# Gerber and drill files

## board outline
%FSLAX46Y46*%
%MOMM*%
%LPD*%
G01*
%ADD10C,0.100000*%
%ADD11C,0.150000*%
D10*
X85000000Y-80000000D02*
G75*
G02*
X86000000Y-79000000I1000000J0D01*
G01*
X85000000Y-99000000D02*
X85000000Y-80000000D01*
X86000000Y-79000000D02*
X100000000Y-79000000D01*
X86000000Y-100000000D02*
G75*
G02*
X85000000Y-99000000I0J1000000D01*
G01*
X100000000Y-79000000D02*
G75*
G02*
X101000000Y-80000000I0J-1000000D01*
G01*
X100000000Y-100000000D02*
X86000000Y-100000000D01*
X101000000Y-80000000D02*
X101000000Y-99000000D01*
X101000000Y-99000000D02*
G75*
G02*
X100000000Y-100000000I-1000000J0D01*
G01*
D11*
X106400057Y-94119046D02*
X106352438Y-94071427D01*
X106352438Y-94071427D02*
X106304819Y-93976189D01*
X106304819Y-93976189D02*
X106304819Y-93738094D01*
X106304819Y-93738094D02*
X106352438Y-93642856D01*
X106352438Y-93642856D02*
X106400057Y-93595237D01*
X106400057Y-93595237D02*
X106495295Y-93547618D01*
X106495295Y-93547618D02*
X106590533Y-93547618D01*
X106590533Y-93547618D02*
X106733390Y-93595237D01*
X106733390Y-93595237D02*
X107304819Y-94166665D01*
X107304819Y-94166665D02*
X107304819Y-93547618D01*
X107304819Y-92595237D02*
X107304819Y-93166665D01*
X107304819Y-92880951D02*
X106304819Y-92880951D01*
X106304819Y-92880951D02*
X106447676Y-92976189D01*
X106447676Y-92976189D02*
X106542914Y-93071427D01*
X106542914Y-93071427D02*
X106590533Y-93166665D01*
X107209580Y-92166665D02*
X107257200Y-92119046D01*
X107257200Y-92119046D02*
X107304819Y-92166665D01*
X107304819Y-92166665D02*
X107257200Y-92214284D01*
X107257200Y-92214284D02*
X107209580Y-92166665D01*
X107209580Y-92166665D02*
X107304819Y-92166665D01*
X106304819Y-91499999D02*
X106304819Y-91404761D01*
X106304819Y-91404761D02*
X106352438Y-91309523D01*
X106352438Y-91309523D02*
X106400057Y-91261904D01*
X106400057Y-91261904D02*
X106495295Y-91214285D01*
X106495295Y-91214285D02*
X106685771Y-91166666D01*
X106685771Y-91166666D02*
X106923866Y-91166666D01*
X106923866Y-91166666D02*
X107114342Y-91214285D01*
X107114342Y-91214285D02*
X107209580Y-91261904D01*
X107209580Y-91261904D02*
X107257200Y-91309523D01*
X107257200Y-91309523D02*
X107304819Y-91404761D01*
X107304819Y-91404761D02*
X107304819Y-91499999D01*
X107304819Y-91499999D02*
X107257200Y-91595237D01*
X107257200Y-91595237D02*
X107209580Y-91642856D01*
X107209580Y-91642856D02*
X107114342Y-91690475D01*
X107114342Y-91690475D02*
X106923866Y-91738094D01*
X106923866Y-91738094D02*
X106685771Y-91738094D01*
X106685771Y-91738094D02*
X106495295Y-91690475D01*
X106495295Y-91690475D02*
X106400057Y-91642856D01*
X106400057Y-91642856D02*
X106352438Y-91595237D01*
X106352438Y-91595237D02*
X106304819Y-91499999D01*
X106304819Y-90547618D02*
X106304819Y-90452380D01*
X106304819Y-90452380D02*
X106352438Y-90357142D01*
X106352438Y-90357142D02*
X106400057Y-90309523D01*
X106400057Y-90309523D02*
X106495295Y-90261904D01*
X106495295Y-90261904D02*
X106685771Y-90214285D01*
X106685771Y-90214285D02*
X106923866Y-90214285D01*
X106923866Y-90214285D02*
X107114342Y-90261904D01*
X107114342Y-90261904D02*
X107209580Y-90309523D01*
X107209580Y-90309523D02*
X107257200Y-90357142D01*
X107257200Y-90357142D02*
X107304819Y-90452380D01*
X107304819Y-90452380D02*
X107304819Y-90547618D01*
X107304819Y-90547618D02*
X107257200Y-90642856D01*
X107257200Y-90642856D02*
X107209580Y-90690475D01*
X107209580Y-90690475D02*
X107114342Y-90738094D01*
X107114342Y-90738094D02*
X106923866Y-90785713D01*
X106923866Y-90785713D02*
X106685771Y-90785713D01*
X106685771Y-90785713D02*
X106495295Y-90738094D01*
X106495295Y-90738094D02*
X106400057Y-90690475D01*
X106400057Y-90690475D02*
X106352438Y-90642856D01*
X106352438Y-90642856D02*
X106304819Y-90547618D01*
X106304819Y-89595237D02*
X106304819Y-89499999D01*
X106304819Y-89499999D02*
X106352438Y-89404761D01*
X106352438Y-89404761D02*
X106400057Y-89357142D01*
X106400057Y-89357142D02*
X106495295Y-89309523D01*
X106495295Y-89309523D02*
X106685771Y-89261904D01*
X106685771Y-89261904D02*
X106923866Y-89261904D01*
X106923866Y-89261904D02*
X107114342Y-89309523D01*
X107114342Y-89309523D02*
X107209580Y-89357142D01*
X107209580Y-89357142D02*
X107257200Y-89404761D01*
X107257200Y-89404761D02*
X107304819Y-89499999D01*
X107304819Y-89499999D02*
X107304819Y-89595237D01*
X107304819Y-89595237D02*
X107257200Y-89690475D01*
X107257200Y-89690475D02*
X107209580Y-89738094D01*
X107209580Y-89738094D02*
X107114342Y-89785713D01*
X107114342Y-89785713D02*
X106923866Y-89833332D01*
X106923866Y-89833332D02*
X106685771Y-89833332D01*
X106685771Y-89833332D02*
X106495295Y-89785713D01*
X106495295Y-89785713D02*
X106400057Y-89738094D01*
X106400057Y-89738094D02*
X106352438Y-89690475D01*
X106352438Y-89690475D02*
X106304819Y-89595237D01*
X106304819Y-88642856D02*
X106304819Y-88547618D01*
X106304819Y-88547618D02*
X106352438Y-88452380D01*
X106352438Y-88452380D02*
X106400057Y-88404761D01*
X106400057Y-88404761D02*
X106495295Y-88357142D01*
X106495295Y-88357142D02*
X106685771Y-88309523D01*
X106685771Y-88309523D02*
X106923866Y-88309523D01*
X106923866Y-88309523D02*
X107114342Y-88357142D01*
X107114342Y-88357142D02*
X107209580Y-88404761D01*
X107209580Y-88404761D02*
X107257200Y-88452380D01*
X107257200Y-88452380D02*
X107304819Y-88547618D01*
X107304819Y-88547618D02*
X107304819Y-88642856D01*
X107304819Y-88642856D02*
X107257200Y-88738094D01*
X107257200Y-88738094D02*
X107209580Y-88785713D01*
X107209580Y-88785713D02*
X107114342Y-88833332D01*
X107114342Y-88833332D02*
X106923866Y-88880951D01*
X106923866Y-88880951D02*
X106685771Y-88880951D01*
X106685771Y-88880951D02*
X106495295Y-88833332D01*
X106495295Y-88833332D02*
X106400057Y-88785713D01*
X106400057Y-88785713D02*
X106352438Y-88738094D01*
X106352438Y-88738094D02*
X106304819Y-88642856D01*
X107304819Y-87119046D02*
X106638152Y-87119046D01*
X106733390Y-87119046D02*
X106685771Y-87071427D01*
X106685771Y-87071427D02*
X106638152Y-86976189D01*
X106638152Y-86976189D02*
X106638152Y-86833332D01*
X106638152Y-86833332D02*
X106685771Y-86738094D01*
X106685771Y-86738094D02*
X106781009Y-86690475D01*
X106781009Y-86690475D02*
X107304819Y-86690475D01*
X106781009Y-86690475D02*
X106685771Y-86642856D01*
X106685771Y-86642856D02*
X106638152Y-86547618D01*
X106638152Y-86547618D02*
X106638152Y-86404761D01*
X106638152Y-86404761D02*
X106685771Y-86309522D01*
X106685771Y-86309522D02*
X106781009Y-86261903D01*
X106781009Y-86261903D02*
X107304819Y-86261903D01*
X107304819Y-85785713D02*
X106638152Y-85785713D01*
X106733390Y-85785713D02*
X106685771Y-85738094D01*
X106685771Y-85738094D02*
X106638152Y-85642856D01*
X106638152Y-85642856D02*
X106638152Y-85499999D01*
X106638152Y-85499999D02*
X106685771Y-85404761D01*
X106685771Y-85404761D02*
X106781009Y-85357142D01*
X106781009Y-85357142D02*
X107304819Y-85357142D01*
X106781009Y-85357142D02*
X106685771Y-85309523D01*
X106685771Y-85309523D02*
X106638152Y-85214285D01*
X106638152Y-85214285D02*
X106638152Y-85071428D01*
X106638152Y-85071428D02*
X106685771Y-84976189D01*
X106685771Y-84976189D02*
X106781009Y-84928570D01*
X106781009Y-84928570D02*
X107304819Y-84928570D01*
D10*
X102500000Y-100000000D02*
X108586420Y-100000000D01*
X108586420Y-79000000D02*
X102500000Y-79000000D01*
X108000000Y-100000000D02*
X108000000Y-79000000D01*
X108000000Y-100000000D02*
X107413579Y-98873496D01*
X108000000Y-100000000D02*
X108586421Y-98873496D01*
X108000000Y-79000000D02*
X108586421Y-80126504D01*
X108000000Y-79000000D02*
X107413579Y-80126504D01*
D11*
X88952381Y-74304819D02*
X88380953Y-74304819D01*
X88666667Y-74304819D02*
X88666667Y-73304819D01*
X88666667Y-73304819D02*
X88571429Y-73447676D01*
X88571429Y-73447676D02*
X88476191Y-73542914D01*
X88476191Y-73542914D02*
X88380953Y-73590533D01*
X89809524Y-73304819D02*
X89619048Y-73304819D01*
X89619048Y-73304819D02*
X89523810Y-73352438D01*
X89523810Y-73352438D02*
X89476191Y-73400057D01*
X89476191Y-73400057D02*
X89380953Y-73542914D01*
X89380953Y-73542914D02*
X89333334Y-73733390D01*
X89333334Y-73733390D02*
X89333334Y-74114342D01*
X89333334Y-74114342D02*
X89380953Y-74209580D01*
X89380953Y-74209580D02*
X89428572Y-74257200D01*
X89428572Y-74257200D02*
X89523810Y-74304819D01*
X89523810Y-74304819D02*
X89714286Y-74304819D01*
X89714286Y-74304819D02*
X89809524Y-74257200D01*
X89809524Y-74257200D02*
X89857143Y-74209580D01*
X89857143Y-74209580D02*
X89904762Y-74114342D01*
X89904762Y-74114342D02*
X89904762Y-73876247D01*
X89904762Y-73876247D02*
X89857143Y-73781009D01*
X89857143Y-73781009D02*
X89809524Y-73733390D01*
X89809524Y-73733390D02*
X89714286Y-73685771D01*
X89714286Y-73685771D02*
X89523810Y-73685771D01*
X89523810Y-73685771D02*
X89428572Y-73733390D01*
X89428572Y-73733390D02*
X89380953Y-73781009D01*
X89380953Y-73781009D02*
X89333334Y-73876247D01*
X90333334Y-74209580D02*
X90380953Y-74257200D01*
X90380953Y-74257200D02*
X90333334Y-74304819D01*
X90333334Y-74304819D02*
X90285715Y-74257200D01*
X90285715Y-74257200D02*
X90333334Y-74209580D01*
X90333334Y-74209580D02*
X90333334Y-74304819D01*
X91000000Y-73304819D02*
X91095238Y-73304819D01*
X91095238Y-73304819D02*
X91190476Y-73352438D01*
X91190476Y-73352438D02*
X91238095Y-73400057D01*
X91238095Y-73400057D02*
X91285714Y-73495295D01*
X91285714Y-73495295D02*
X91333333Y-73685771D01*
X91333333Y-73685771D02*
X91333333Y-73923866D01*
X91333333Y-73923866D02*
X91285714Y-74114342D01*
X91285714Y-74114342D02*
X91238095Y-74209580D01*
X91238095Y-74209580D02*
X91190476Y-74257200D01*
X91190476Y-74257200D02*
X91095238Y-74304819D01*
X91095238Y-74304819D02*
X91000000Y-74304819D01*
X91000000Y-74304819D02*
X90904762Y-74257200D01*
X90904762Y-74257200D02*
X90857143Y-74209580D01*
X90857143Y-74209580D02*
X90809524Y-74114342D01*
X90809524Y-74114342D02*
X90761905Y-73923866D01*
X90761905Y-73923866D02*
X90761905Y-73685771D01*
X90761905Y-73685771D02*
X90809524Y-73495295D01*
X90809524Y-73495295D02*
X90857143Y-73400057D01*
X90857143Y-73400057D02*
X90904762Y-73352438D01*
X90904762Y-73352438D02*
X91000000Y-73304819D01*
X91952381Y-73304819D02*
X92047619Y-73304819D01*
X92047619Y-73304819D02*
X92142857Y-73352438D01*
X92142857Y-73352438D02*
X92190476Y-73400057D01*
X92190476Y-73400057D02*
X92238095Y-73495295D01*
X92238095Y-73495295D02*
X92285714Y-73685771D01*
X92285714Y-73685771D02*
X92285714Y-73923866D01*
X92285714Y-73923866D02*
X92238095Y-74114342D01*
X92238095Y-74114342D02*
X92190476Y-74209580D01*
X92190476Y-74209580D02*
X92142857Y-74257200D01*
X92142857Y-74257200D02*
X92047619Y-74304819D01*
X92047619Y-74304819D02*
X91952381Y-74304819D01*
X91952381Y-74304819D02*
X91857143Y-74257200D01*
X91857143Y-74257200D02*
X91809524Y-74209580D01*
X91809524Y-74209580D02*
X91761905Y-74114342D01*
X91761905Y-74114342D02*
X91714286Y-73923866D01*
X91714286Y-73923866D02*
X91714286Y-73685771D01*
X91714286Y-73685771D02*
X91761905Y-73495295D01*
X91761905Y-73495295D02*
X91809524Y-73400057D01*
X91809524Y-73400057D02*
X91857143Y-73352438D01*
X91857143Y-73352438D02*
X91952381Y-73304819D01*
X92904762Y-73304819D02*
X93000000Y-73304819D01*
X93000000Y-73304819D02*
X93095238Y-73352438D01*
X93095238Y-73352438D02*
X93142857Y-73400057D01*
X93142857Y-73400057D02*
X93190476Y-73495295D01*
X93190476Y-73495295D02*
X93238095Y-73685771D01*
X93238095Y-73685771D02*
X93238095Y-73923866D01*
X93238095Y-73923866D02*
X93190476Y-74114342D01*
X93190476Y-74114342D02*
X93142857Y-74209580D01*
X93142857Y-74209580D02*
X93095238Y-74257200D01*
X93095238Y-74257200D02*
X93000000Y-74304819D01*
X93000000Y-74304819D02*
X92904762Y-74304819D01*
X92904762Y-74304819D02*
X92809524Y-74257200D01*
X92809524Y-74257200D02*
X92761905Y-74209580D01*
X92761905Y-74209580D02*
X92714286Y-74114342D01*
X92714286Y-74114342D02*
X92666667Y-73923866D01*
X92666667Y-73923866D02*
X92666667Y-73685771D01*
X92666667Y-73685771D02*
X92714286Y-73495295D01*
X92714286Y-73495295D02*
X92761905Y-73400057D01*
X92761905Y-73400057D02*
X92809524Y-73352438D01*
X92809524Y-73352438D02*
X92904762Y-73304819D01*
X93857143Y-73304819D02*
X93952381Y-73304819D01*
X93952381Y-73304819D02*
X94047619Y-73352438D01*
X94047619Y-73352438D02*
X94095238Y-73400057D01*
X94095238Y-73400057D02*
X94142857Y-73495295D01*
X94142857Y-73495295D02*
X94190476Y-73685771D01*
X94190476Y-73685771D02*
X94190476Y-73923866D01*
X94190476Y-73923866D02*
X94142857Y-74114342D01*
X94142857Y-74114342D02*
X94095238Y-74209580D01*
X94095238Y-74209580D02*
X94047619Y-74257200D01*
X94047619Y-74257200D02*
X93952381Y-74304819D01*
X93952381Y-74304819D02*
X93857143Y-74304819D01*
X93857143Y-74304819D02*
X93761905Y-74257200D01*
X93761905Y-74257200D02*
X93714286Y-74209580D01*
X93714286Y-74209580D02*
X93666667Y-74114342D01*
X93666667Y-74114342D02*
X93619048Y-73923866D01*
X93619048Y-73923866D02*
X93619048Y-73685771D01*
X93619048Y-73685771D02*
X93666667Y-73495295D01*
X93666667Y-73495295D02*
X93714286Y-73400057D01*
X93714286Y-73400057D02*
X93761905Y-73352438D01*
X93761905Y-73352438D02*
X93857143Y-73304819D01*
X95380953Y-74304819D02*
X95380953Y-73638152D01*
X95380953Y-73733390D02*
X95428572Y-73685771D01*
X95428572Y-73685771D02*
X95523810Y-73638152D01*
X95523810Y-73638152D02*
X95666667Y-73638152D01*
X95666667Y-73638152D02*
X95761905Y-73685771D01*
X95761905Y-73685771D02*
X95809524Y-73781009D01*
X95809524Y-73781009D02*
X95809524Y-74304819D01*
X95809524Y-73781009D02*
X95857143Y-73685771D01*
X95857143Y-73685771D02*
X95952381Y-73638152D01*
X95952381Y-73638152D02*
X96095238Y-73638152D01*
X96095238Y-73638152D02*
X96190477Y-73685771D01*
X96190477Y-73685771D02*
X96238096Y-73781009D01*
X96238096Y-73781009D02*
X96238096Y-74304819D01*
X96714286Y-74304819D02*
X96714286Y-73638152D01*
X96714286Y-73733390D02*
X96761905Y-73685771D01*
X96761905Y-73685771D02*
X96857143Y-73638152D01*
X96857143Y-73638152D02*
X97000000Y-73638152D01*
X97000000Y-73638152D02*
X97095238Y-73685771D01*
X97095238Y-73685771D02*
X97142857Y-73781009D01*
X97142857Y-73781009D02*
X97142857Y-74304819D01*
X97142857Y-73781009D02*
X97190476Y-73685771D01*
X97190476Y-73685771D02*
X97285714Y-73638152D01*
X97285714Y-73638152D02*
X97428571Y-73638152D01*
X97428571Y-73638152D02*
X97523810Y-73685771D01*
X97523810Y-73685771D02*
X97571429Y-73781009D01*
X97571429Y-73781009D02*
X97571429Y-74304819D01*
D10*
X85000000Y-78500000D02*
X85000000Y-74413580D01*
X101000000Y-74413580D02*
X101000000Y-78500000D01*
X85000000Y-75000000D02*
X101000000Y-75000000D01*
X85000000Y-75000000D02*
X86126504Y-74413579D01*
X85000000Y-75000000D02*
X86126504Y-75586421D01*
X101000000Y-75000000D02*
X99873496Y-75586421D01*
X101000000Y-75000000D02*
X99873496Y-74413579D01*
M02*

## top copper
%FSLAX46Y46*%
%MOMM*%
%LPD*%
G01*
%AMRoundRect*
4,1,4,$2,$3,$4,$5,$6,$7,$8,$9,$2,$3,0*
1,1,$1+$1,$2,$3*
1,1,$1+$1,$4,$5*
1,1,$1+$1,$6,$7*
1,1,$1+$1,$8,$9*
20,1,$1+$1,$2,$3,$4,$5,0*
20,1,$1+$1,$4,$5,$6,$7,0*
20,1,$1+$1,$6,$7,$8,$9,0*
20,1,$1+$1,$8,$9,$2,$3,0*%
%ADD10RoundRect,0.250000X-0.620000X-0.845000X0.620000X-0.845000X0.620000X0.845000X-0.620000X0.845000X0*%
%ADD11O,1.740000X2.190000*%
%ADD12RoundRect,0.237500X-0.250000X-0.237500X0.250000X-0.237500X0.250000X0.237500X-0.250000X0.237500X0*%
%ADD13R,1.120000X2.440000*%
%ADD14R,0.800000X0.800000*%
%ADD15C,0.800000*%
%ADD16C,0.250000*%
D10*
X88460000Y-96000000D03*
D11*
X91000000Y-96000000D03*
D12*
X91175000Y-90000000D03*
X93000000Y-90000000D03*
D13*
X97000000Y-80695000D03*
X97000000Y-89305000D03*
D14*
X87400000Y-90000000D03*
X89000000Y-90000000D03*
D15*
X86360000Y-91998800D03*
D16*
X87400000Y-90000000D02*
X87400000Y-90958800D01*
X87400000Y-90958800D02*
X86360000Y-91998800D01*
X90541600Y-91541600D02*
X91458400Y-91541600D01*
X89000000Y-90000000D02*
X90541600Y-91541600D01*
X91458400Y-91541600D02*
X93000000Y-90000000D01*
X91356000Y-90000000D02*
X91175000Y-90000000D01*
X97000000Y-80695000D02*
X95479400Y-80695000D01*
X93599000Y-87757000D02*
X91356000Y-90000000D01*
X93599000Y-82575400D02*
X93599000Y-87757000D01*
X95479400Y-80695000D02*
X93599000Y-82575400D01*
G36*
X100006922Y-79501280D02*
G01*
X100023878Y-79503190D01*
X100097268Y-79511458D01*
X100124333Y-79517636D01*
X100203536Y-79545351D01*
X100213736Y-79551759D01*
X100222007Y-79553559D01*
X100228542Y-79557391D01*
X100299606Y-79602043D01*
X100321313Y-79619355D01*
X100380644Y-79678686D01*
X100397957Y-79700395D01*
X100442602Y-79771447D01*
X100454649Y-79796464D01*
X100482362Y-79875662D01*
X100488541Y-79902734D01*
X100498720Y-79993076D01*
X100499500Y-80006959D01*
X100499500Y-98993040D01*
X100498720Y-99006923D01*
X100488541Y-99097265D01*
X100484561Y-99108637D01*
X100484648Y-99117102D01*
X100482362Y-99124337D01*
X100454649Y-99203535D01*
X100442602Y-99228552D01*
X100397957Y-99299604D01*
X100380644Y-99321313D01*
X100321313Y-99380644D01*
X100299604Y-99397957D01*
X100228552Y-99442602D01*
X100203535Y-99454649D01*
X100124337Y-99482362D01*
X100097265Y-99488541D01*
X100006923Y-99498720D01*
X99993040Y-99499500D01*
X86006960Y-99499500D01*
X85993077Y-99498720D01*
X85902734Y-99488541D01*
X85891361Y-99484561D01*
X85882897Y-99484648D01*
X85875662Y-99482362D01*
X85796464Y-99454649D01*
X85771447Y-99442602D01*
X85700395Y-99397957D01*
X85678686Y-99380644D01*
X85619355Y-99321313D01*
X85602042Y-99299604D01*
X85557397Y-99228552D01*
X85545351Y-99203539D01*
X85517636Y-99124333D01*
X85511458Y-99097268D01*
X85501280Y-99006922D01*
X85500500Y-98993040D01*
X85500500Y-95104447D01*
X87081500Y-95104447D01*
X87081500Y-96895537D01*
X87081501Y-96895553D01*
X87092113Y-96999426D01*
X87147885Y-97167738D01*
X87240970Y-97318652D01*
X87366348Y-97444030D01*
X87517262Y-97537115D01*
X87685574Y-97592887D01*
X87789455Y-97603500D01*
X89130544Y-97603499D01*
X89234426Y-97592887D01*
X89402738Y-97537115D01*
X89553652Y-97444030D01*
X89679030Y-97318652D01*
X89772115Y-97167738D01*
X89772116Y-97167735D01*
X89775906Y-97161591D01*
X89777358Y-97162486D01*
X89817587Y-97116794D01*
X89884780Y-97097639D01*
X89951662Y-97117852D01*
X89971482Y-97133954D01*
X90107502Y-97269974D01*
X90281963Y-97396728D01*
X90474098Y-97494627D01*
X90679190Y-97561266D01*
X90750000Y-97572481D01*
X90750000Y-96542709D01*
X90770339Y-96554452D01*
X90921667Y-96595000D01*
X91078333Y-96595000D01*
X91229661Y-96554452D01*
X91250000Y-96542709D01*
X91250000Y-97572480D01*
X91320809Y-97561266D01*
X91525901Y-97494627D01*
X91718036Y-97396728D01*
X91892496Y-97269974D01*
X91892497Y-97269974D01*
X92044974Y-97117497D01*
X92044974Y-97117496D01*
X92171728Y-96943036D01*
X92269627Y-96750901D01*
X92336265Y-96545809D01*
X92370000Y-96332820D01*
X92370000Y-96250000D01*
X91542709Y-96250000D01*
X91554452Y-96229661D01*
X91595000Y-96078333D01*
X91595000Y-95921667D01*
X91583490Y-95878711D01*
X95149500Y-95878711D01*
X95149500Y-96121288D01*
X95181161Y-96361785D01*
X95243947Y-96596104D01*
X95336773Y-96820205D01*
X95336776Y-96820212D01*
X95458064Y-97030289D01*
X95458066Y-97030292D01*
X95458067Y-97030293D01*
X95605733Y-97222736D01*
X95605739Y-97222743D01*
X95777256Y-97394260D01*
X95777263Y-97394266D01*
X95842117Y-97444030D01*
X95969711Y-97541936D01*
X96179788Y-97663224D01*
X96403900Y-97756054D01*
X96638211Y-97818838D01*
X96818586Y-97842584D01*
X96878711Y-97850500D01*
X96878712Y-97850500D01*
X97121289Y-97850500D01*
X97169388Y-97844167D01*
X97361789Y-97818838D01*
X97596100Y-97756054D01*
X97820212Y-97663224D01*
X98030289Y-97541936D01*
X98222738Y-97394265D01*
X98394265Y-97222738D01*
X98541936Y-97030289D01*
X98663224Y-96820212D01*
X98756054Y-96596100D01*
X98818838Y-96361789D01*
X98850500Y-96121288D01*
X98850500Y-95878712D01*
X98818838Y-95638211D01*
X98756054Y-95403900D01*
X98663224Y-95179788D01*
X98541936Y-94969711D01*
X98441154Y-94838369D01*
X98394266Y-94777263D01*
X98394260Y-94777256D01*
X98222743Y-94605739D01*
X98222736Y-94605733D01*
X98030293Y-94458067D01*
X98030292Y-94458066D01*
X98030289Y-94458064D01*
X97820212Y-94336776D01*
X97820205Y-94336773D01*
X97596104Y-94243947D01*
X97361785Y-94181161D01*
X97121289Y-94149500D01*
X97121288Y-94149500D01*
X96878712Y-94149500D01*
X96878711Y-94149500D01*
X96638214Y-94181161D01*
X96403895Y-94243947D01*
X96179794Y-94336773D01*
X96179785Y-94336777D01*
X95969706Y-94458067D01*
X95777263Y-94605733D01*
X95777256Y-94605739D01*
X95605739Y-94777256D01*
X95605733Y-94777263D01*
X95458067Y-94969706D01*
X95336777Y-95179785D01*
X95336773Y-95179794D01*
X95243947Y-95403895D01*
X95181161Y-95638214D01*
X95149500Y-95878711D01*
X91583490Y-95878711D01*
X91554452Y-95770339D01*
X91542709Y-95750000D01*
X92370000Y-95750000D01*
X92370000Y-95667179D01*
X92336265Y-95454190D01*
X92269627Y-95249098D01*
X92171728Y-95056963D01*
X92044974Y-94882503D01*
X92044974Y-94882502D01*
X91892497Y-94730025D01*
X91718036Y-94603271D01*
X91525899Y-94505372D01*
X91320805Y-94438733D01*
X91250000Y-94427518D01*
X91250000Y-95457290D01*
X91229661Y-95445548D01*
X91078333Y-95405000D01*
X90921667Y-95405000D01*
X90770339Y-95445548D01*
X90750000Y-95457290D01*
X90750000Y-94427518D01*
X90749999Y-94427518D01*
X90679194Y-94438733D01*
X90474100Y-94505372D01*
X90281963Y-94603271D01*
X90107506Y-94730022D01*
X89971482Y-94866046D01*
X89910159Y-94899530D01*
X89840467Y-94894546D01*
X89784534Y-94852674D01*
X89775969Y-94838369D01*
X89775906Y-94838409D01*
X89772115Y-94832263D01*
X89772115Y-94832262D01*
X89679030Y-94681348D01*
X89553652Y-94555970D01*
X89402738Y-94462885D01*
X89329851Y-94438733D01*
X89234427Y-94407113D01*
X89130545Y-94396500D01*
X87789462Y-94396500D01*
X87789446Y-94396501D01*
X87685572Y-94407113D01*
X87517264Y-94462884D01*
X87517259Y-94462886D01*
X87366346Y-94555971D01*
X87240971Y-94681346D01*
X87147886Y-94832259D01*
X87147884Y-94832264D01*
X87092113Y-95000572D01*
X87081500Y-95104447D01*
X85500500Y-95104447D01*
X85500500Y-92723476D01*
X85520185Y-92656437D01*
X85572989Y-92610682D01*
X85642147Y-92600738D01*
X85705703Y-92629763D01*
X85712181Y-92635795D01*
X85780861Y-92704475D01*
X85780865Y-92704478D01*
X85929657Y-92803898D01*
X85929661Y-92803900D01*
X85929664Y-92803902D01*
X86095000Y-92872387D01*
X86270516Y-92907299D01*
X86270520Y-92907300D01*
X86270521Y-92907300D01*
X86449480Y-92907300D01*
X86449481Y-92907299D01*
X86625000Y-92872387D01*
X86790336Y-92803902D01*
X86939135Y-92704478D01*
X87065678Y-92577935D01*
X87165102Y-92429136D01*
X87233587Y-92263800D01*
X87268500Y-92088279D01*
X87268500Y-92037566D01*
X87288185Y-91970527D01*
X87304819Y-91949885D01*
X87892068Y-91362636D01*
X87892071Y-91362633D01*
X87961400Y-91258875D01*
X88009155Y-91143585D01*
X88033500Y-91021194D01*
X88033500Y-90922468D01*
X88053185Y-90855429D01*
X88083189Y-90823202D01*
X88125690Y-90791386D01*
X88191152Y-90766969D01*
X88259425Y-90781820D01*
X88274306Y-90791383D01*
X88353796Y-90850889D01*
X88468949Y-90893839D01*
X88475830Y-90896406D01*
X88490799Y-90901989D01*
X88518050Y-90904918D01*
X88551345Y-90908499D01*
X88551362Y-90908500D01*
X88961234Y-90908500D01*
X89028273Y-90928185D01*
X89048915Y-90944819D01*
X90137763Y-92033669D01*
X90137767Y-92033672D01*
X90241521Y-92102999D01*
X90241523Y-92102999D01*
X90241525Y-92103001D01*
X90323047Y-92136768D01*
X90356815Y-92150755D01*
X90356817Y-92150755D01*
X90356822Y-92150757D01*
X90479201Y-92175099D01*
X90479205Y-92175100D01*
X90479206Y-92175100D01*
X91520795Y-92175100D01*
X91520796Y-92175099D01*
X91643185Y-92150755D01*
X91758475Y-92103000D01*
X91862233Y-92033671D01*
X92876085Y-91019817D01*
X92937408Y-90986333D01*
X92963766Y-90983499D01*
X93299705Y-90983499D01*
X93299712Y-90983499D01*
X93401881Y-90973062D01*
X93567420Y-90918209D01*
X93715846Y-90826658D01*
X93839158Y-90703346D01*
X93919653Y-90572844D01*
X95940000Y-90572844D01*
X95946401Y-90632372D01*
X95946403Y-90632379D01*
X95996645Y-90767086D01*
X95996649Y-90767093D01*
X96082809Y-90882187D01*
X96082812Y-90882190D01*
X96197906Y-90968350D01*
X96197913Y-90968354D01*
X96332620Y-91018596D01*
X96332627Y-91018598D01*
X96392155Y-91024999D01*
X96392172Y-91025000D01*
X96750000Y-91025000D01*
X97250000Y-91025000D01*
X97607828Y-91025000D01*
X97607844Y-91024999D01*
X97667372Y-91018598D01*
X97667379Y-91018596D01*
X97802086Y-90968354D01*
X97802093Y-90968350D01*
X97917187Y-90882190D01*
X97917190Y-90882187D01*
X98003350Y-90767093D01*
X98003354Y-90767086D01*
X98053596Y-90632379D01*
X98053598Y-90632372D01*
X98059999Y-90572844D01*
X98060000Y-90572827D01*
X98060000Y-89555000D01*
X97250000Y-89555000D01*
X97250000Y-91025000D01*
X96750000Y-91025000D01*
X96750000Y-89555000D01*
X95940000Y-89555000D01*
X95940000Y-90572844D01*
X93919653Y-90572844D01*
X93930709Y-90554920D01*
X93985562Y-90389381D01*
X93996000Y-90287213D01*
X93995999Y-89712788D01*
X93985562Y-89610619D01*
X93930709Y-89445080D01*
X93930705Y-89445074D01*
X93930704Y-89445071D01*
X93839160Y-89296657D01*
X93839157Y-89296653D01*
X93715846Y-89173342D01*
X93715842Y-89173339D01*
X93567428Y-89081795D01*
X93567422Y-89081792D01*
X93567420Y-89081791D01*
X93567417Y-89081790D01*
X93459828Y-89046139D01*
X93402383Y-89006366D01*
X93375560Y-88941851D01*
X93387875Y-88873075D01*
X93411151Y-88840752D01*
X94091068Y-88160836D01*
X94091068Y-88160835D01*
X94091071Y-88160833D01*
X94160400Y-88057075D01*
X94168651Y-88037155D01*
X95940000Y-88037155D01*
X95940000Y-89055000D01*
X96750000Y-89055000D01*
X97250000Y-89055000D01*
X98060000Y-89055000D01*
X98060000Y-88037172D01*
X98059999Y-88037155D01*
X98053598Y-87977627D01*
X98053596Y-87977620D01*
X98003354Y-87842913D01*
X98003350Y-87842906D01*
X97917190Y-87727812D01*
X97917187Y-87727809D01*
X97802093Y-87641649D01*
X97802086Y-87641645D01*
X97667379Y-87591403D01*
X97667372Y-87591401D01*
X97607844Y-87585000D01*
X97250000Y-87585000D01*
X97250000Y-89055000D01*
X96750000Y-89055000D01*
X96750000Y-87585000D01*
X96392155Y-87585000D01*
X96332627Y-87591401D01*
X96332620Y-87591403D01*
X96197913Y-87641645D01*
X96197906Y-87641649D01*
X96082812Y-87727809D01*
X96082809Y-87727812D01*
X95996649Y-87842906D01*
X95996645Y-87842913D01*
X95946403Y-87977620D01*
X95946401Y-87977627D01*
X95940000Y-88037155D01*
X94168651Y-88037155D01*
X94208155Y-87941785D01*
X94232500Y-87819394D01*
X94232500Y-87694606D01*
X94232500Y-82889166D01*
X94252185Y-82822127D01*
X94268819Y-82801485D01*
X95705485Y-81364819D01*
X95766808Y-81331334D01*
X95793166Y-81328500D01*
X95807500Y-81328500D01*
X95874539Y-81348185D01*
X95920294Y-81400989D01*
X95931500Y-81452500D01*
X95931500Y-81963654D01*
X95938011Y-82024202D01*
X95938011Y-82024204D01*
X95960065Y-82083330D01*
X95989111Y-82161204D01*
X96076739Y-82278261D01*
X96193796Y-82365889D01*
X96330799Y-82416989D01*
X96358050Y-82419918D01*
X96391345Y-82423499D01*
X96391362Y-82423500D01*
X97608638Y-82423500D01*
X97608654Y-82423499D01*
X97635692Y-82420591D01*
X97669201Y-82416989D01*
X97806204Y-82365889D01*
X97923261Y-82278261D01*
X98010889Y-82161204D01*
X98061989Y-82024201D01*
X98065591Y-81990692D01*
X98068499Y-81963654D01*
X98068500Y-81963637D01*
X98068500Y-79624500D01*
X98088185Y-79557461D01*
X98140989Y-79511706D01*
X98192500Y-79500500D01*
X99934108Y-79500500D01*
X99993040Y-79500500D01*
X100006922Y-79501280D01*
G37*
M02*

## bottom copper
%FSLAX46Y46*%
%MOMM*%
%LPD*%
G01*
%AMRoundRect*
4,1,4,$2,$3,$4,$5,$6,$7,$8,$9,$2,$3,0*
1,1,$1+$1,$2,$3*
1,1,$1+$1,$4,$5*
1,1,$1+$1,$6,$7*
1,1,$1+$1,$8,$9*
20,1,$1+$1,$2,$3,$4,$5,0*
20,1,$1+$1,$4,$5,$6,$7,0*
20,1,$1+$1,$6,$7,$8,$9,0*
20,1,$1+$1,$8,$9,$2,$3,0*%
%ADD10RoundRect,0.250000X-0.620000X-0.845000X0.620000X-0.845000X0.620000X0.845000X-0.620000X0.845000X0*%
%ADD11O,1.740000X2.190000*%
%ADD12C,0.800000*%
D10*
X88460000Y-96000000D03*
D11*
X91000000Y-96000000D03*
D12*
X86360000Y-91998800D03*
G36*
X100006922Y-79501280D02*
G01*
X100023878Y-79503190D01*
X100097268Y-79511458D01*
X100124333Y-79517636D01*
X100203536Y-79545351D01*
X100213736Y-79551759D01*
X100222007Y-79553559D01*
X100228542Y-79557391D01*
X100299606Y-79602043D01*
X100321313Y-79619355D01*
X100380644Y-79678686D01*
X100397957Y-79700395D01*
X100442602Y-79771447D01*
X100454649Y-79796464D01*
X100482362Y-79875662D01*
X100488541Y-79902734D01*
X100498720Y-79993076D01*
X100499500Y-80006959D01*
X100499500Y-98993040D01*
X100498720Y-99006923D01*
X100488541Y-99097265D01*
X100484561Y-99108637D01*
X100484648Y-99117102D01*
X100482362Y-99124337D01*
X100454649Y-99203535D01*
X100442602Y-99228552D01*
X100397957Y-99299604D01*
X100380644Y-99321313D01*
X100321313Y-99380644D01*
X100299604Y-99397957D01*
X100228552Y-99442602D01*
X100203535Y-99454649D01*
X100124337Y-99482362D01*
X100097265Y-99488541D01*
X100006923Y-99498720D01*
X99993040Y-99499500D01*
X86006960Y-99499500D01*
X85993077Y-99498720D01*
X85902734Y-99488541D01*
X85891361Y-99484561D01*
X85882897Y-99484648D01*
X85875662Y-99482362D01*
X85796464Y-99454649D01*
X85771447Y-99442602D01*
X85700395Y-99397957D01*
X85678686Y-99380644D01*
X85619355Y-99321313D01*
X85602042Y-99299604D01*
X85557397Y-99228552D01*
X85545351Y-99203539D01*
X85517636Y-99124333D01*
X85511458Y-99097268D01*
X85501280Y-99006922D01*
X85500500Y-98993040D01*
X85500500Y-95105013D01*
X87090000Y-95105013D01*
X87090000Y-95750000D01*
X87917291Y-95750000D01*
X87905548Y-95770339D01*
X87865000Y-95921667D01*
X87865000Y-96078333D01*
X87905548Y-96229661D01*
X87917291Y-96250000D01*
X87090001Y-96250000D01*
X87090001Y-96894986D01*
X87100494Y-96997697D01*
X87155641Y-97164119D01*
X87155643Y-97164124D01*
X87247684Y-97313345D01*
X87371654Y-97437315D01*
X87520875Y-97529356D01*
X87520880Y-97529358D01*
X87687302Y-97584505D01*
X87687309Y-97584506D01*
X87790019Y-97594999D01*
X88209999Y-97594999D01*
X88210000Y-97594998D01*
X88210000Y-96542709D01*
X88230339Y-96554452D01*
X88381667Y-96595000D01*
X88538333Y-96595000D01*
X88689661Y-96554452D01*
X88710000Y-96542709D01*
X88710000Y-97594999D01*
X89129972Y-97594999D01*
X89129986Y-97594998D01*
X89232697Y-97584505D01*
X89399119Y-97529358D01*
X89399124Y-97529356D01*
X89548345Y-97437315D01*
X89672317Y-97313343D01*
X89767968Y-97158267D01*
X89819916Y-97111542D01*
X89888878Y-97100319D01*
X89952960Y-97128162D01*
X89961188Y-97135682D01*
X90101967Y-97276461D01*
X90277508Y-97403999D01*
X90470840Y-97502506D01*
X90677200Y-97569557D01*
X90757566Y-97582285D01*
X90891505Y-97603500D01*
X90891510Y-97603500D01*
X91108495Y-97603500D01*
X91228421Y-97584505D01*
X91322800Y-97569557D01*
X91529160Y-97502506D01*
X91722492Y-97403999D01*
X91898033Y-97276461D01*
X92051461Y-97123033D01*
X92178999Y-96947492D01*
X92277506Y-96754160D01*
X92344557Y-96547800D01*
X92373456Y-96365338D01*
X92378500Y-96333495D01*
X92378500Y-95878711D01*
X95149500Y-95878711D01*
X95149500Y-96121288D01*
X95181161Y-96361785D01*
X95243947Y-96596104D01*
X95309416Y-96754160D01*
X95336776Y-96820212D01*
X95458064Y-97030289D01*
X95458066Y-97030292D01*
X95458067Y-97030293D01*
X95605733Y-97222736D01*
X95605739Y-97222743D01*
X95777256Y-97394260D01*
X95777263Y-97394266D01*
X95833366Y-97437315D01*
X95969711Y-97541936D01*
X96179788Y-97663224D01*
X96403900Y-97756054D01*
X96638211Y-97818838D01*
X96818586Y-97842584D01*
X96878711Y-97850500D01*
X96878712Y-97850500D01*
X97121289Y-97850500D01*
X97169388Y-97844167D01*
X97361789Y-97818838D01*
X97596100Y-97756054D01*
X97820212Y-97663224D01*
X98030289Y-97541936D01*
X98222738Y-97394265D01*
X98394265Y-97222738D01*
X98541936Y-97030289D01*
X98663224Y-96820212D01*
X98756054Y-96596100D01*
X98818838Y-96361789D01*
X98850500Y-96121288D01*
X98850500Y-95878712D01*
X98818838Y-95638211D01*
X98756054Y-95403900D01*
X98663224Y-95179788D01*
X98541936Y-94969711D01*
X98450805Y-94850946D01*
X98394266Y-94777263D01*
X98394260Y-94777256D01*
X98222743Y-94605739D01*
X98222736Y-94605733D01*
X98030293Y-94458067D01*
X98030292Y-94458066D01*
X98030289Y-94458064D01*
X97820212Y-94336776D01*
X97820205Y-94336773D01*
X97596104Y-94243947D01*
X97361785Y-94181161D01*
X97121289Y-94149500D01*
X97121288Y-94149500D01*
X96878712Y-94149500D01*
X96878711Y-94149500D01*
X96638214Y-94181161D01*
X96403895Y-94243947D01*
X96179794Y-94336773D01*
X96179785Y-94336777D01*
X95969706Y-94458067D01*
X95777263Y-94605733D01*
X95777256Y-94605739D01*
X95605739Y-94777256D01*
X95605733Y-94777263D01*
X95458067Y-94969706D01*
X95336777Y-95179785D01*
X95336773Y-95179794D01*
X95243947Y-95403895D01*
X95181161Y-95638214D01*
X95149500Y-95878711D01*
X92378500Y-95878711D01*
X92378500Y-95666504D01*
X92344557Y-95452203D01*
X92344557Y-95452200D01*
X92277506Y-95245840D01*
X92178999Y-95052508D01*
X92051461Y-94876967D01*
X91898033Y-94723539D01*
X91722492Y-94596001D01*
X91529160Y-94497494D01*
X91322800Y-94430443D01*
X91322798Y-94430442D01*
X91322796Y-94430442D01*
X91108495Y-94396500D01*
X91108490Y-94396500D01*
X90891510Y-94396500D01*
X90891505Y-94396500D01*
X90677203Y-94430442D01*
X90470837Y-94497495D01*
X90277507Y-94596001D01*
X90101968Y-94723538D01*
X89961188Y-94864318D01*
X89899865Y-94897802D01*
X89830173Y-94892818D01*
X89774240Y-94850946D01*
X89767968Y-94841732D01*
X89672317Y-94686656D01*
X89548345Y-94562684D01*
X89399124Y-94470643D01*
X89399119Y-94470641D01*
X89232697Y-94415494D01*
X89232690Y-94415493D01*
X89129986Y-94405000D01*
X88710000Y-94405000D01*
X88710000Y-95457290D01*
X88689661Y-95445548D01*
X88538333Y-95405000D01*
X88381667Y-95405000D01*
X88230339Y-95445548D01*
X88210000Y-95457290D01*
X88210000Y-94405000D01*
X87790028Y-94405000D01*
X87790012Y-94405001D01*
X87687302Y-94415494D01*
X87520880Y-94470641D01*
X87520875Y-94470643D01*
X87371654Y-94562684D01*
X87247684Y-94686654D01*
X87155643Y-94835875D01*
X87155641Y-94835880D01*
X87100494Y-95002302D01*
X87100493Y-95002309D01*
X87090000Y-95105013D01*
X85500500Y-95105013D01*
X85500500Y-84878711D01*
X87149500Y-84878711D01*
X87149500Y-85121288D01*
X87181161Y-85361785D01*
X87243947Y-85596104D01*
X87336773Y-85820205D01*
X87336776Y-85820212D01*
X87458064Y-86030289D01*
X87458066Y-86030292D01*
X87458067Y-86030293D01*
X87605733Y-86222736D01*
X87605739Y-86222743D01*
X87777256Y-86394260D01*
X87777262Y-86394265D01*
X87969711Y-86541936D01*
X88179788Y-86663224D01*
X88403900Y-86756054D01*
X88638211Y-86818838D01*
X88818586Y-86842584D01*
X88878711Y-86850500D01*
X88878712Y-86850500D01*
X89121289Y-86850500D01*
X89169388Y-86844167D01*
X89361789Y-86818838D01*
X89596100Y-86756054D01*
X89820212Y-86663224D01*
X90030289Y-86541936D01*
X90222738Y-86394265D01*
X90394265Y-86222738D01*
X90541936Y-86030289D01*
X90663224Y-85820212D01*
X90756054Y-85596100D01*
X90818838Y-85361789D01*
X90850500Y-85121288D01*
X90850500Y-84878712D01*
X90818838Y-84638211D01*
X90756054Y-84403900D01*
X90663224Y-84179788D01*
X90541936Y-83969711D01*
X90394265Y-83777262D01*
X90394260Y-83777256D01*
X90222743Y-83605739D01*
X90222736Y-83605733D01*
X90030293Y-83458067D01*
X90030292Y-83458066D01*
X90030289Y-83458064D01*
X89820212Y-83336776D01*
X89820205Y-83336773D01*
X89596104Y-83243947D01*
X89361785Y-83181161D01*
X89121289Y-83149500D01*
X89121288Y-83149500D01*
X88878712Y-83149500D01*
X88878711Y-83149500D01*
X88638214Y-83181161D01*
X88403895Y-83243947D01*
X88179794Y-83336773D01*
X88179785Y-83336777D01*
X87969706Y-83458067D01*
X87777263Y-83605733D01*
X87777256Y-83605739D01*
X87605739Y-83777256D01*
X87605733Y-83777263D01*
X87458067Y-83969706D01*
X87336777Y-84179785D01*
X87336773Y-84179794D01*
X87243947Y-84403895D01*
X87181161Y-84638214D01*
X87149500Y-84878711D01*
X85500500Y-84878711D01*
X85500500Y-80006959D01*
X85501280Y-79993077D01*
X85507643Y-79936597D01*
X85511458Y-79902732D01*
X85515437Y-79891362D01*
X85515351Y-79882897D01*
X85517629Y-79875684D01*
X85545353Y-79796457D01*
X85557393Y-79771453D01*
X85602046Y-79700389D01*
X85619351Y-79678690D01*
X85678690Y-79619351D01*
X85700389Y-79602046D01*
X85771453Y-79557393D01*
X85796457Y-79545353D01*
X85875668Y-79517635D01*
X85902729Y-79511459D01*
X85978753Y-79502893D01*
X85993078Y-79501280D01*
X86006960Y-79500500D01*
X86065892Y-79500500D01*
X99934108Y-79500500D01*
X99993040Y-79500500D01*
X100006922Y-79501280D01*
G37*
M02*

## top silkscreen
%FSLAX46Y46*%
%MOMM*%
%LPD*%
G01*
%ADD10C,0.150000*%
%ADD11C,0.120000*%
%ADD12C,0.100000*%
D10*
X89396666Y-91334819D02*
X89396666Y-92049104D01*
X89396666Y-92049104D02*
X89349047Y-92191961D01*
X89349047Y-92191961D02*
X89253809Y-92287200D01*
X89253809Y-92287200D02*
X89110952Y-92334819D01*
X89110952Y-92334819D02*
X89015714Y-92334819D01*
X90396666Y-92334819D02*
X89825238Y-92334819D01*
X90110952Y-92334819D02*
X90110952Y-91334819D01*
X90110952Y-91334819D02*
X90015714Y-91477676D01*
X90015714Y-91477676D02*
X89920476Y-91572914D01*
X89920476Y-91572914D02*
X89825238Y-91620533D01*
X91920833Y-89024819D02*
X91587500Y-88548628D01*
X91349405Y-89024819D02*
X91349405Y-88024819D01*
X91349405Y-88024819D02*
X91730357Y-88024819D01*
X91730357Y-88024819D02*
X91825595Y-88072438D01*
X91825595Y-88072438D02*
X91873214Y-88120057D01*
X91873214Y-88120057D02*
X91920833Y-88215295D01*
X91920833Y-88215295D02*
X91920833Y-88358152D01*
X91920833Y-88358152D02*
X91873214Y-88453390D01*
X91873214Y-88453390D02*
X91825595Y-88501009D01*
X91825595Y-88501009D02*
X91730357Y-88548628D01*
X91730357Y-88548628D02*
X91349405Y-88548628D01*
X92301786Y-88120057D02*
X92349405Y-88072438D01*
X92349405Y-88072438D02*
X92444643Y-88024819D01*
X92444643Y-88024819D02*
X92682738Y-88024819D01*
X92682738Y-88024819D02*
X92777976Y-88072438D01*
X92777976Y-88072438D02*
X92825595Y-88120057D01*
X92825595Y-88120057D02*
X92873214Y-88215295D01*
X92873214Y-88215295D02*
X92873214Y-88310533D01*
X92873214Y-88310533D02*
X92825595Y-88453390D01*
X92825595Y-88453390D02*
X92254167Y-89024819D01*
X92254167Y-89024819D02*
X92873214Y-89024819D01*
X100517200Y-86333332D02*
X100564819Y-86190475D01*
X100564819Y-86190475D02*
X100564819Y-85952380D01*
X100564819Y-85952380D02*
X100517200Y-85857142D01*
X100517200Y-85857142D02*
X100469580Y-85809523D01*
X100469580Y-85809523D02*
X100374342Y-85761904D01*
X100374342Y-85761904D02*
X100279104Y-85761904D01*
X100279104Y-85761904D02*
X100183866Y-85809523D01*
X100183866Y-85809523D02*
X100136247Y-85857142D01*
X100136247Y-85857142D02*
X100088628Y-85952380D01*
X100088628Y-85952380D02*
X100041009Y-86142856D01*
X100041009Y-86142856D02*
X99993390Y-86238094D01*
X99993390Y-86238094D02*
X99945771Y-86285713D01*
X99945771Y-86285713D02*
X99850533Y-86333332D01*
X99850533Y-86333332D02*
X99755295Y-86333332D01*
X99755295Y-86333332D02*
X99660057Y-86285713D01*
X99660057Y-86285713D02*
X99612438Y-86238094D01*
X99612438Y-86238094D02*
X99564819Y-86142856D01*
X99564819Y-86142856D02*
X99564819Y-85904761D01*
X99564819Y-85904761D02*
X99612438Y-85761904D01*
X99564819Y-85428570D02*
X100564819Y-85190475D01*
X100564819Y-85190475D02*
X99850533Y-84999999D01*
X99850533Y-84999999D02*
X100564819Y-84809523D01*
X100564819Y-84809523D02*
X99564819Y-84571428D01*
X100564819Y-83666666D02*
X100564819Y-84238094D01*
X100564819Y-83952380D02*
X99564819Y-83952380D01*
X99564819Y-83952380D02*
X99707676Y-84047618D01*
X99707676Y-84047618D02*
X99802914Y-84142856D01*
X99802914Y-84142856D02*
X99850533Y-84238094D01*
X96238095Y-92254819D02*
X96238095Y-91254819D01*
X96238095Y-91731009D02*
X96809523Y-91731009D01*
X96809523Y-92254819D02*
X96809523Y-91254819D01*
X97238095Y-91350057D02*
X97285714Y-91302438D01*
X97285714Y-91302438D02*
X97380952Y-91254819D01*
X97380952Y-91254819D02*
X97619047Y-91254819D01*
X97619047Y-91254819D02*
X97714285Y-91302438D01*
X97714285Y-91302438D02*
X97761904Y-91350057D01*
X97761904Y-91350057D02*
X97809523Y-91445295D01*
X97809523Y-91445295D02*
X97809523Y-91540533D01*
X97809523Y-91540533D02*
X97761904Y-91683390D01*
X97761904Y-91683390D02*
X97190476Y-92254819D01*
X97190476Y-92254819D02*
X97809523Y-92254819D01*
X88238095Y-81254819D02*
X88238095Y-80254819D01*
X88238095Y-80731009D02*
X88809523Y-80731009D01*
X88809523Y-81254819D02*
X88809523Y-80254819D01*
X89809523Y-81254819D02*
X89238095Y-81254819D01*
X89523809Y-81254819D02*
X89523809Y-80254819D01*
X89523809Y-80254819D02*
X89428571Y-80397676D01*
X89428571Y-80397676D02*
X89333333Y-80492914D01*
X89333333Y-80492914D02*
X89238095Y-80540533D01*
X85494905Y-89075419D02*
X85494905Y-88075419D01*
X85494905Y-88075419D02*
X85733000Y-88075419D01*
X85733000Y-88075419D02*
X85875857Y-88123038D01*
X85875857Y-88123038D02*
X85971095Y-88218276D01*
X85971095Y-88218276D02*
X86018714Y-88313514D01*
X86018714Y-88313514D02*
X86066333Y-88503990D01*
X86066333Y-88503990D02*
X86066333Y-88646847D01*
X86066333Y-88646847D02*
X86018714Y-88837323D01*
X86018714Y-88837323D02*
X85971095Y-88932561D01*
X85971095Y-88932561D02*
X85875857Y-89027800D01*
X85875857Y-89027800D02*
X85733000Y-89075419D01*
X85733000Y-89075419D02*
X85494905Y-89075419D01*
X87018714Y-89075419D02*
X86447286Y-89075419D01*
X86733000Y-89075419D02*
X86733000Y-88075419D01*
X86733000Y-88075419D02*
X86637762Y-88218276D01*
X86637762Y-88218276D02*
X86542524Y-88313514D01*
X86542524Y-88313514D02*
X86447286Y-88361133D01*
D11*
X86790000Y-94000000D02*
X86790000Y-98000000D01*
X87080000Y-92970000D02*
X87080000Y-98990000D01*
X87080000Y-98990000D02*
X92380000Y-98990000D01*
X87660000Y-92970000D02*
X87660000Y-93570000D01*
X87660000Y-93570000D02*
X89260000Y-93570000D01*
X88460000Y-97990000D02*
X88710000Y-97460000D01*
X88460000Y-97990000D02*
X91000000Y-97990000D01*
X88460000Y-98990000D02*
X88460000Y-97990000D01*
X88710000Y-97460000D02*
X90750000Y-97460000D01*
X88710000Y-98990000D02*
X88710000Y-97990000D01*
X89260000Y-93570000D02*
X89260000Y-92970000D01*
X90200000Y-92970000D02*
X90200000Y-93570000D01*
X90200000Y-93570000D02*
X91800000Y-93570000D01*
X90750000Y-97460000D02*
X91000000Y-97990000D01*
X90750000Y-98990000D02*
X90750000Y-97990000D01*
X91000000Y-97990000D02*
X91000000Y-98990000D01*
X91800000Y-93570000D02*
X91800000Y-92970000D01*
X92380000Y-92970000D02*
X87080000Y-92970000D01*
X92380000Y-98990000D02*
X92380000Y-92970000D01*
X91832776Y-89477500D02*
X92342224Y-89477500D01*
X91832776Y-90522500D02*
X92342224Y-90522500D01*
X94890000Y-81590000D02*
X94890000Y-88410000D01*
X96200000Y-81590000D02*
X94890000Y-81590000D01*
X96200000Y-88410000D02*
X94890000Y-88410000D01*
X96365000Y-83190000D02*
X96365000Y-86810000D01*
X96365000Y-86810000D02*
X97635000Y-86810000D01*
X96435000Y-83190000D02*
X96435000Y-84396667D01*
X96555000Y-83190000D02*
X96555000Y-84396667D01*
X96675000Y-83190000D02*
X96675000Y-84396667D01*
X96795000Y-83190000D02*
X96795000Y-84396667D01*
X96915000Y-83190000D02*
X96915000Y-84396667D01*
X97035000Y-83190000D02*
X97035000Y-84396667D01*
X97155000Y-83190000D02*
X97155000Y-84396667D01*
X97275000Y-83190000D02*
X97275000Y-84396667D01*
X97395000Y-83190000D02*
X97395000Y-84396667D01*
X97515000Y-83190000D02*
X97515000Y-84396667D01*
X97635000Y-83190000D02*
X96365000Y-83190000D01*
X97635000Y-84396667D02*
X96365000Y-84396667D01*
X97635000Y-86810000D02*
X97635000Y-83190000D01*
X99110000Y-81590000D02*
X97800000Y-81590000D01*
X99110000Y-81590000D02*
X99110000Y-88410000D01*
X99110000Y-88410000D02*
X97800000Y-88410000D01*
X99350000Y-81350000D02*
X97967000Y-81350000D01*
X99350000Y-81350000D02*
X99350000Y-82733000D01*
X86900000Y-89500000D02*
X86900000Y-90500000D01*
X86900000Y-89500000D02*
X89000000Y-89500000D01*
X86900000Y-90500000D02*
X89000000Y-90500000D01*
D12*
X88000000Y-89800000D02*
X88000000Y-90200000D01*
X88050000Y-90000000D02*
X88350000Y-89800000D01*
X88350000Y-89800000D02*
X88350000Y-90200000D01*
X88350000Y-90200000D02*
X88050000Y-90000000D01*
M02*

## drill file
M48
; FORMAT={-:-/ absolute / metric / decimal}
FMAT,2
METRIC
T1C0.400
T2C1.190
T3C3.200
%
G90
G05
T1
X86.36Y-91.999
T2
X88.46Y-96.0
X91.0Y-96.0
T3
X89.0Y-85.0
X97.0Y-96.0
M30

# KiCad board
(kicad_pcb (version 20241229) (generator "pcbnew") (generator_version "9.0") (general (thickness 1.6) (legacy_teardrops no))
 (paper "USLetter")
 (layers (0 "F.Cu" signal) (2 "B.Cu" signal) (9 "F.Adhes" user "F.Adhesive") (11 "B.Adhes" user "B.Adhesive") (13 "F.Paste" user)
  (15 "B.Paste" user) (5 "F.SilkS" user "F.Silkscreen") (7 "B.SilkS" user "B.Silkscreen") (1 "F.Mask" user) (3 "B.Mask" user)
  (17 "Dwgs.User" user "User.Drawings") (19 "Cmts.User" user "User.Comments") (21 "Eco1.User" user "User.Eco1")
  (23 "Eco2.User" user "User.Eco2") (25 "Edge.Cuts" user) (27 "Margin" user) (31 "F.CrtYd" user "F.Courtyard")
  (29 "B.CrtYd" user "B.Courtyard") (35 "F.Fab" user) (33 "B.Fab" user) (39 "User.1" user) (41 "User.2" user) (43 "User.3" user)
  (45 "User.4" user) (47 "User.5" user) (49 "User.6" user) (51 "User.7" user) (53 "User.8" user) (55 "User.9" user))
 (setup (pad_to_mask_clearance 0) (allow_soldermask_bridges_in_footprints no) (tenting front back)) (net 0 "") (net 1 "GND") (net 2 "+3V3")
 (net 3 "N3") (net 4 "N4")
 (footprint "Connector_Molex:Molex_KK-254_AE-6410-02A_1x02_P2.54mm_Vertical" (layer "F.Cu") (at 88.46 96)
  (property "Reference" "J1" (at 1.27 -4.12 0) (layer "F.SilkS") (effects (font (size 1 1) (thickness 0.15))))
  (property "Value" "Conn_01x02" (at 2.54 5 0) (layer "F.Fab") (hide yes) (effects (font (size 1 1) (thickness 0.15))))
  (fp_line (start -1.67 -2) (end -1.67 2) (stroke (width 0.12) (type solid)) (layer "F.SilkS"))
  (fp_line (start -1.38 -3.03) (end -1.38 2.99) (stroke (width 0.12) (type solid)) (layer "F.SilkS"))
  (fp_line (start -1.38 2.99) (end 3.92 2.99) (stroke (width 0.12) (type solid)) (layer "F.SilkS"))
  (fp_line (start -0.8 -3.03) (end -0.8 -2.43) (stroke (width 0.12) (type solid)) (layer "F.SilkS"))
  (fp_line (start -0.8 -2.43) (end 0.8 -2.43) (stroke (width 0.12) (type solid)) (layer "F.SilkS"))
  (fp_line (start 0 1.99) (end 0.25 1.46) (stroke (width 0.12) (type solid)) (layer "F.SilkS"))
  (fp_line (start 0 1.99) (end 2.54 1.99) (stroke (width 0.12) (type solid)) (layer "F.SilkS"))
  (fp_line (start 0 2.99) (end 0 1.99) (stroke (width 0.12) (type solid)) (layer "F.SilkS"))
  (fp_line (start 0.25 1.46) (end 2.29 1.46) (stroke (width 0.12) (type solid)) (layer "F.SilkS"))
  (fp_line (start 0.25 2.99) (end 0.25 1.99) (stroke (width 0.12) (type solid)) (layer "F.SilkS"))
  (fp_line (start 0.8 -2.43) (end 0.8 -3.03) (stroke (width 0.12) (type solid)) (layer "F.SilkS"))
  (fp_line (start 1.74 -3.03) (end 1.74 -2.43) (stroke (width 0.12) (type solid)) (layer "F.SilkS"))
  (fp_line (start 1.74 -2.43) (end 3.34 -2.43) (stroke (width 0.12) (type solid)) (layer "F.SilkS"))
  (fp_line (start 2.29 1.46) (end 2.54 1.99) (stroke (width 0.12) (type solid)) (layer "F.SilkS"))
  (fp_line (start 2.29 2.99) (end 2.29 1.99) (stroke (width 0.12) (type solid)) (layer "F.SilkS"))
  (fp_line (start 2.54 1.99) (end 2.54 2.99) (stroke (width 0.12) (type solid)) (layer "F.SilkS"))
  (fp_line (start 3.34 -2.43) (end 3.34 -3.03) (stroke (width 0.12) (type solid)) (layer "F.SilkS"))
  (fp_line (start 3.92 -3.03) (end -1.38 -3.03) (stroke (width 0.12) (type solid)) (layer "F.SilkS"))
  (fp_line (start 3.92 2.99) (end 3.92 -3.03) (stroke (width 0.12) (type solid)) (layer "F.SilkS"))
  (pad "1" thru_hole roundrect (at 0 0) (size 1.74 2.19) (drill 1.19) (layers "*.Cu" "*.Mask") (remove_unused_layers no)
   (roundrect_rratio 0.143678) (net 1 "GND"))
  (pad "2" thru_hole oval (at 2.54 0) (size 1.74 2.19) (drill 1.19) (layers "*.Cu" "*.Mask") (remove_unused_layers no) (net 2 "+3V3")))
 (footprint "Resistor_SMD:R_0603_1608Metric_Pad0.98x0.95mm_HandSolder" (layer "F.Cu") (at 92.0875 90)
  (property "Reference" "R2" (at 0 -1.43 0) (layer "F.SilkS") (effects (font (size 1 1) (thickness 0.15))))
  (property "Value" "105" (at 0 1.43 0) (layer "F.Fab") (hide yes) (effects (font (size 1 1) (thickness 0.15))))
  (fp_line (start -0.254724 -0.5225) (end 0.254724 -0.5225) (stroke (width 0.12) (type solid)) (layer "F.SilkS"))
  (fp_line (start -0.254724 0.5225) (end 0.254724 0.5225) (stroke (width 0.12) (type solid)) (layer "F.SilkS"))
  (pad "1" smd roundrect (at -0.9125 0) (size 0.975 0.95) (layers "F.Cu" "F.Mask" "F.Paste") (roundrect_rratio 0.25) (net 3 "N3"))
  (pad "2" smd roundrect (at 0.9125 0) (size 0.975 0.95) (layers "F.Cu" "F.Mask" "F.Paste") (roundrect_rratio 0.25) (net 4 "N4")))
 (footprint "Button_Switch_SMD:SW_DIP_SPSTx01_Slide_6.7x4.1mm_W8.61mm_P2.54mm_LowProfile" (layer "F.Cu") (at 97 85 -90)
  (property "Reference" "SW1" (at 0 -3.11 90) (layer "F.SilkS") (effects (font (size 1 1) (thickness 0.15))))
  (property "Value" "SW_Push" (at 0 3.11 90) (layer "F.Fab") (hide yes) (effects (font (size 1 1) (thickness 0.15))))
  (fp_line (start -3.41 2.11) (end 3.41 2.11) (stroke (width 0.12) (type solid)) (layer "F.SilkS"))
  (fp_line (start -3.41 0.8) (end -3.41 2.11) (stroke (width 0.12) (type solid)) (layer "F.SilkS"))
  (fp_line (start 3.41 0.8) (end 3.41 2.11) (stroke (width 0.12) (type solid)) (layer "F.SilkS"))
  (fp_line (start -1.81 0.635) (end 1.81 0.635) (stroke (width 0.12) (type solid)) (layer "F.SilkS"))
  (fp_line (start 1.81 0.635) (end 1.81 -0.635) (stroke (width 0.12) (type solid)) (layer "F.SilkS"))
  (fp_line (start -1.81 0.565) (end -0.603333 0.565) (stroke (width 0.12) (type solid)) (layer "F.SilkS"))
  (fp_line (start -1.81 0.445) (end -0.603333 0.445) (stroke (width 0.12) (type solid)) (layer "F.SilkS"))
  (fp_line (start -1.81 0.325) (end -0.603333 0.325) (stroke (width 0.12) (type solid)) (layer "F.SilkS"))
  (fp_line (start -1.81 0.205) (end -0.603333 0.205) (stroke (width 0.12) (type solid)) (layer "F.SilkS"))
  (fp_line (start -1.81 0.085) (end -0.603333 0.085) (stroke (width 0.12) (type solid)) (layer "F.SilkS"))
  (fp_line (start -1.81 -0.035) (end -0.603333 -0.035) (stroke (width 0.12) (type solid)) (layer "F.SilkS"))
  (fp_line (start -1.81 -0.155) (end -0.603333 -0.155) (stroke (width 0.12) (type solid)) (layer "F.SilkS"))
  (fp_line (start -1.81 -0.275) (end -0.603333 -0.275) (stroke (width 0.12) (type solid)) (layer "F.SilkS"))
  (fp_line (start -1.81 -0.395) (end -0.603333 -0.395) (stroke (width 0.12) (type solid)) (layer "F.SilkS"))
  (fp_line (start -1.81 -0.515) (end -0.603333 -0.515) (stroke (width 0.12) (type solid)) (layer "F.SilkS"))
  (fp_line (start -1.81 -0.635) (end -1.81 0.635) (stroke (width 0.12) (type solid)) (layer "F.SilkS"))
  (fp_line (start -0.603333 -0.635) (end -0.603333 0.635) (stroke (width 0.12) (type solid)) (layer "F.SilkS"))
  (fp_line (start 1.81 -0.635) (end -1.81 -0.635) (stroke (width 0.12) (type solid)) (layer "F.SilkS"))
  (fp_line (start -3.41 -2.11) (end -3.41 -0.8) (stroke (width 0.12) (type solid)) (layer "F.SilkS"))
  (fp_line (start -3.41 -2.11) (end 3.41 -2.11) (stroke (width 0.12) (type solid)) (layer "F.SilkS"))
  (fp_line (start 3.41 -2.11) (end 3.41 -0.8) (stroke (width 0.12) (type solid)) (layer "F.SilkS"))
  (fp_line (start -3.65 -2.35) (end -3.65 -0.967) (stroke (width 0.12) (type solid)) (layer "F.SilkS"))
  (fp_line (start -3.65 -2.35) (end -2.267 -2.35) (stroke (width 0.12) (type solid)) (layer "F.SilkS"))
  (pad "1" smd rect (at -4.305 0 270) (size 2.44 1.12) (layers "F.Cu" "F.Mask" "F.Paste") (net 3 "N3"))
  (pad "2" smd rect (at 4.305 0 270) (size 2.44 1.12) (layers "F.Cu" "F.Mask" "F.Paste") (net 2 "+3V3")))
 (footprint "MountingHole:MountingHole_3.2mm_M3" (layer "F.Cu") (at 97 96)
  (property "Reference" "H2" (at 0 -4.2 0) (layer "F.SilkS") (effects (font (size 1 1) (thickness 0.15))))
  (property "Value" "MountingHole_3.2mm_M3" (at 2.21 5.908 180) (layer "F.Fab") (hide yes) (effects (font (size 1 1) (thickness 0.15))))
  (pad "" np_thru_hole circle (at 0 0) (size 3.2 3.2) (drill 3.2) (layers "*.Cu" "*.Mask")))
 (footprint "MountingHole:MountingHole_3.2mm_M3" (layer "F.Cu") (at 89 85)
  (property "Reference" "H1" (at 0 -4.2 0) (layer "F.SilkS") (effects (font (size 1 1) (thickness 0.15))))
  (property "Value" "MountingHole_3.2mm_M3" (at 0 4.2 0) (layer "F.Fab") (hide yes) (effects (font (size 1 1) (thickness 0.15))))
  (pad "" np_thru_hole circle (at 0 0) (size 3.2 3.2) (drill 3.2) (layers "*.Cu" "*.Mask")))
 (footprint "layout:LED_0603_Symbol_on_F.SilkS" (layer "F.Cu") (at 88.2 90)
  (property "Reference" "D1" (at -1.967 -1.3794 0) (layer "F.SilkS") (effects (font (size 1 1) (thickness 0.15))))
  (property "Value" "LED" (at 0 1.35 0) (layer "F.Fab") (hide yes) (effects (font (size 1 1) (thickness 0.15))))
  (fp_line (start -1.3 -0.5) (end -1.3 0.5) (stroke (width 0.12) (type solid)) (layer "F.SilkS"))
  (fp_line (start -1.3 -0.5) (end 0.8 -0.5) (stroke (width 0.12) (type solid)) (layer "F.SilkS"))
  (fp_line (start -1.3 0.5) (end 0.8 0.5) (stroke (width 0.12) (type solid)) (layer "F.SilkS"))
  (fp_line (start -0.2 -0.2) (end -0.2 0.2) (stroke (width 0.1) (type solid)) (layer "F.SilkS"))
  (fp_line (start -0.15 0) (end 0.15 -0.2) (stroke (width 0.1) (type solid)) (layer "F.SilkS"))
  (fp_line (start 0.15 -0.2) (end 0.15 0.2) (stroke (width 0.1) (type solid)) (layer "F.SilkS"))
  (fp_line (start 0.15 0.2) (end -0.15 0) (stroke (width 0.1) (type solid)) (layer "F.SilkS"))
  (pad "1" smd rect (at -0.8 0 180) (size 0.8 0.8) (layers "F.Cu" "F.Mask" "F.Paste") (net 1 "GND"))
  (pad "2" smd rect (at 0.8 0 180) (size 0.8 0.8) (layers "F.Cu" "F.Mask" "F.Paste") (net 4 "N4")))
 (gr_arc (start 85 80) (mid 85.292893 79.292893) (end 86 79) (stroke (width 0.1) (type default)) (layer "Edge.Cuts"))
 (gr_line (start 85 99) (end 85 80) (stroke (width 0.1) (type default)) (layer "Edge.Cuts"))
 (gr_line (start 86 79) (end 100 79) (stroke (width 0.1) (type default)) (layer "Edge.Cuts"))
 (gr_arc (start 86 100) (mid 85.292893 99.707107) (end 85 99) (stroke (width 0.1) (type default)) (layer "Edge.Cuts"))
 (gr_arc (start 100 79) (mid 100.707107 79.292893) (end 101 80) (stroke (width 0.1) (type default)) (layer "Edge.Cuts"))
 (gr_line (start 100 100) (end 86 100) (stroke (width 0.1) (type default)) (layer "Edge.Cuts"))
 (gr_line (start 101 80) (end 101 99) (stroke (width 0.1) (type default)) (layer "Edge.Cuts"))
 (gr_arc (start 101 99) (mid 100.707107 99.707107) (end 100 100) (stroke (width 0.1) (type default)) (layer "Edge.Cuts"))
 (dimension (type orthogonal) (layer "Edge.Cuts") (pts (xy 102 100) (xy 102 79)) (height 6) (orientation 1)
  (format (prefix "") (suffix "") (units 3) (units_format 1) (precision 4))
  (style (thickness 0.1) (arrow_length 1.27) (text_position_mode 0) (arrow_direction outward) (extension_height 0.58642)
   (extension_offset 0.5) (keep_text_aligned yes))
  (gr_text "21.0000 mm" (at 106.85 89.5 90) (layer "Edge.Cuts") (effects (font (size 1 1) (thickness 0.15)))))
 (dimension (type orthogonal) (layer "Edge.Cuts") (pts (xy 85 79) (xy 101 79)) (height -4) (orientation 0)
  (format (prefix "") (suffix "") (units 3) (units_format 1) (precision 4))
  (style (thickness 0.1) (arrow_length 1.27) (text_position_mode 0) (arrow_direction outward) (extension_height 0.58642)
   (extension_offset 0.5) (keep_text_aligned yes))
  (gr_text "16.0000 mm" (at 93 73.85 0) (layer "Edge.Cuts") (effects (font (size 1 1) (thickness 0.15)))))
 (segment (start 87.4 90) (end 87.4 90.9588) (width 0.25) (layer "F.Cu") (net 1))
 (segment (start 87.4 90.9588) (end 86.36 91.9988) (width 0.25) (layer "F.Cu") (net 1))
 (via (at 86.36 91.9988) (size 0.8) (drill 0.4) (layers "F.Cu" "B.Cu") (free yes) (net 1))
 (segment (start 90.5416 91.5416) (end 91.4584 91.5416) (width 0.25) (layer "F.Cu") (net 4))
 (segment (start 89 90) (end 90.5416 91.5416) (width 0.25) (layer "F.Cu") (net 4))
 (segment (start 91.4584 91.5416) (end 93 90) (width 0.25) (layer "F.Cu") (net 4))
 (segment (start 91.356 90) (end 91.175 90) (width 0.25) (layer "F.Cu") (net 3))
 (segment (start 97 80.695) (end 95.4794 80.695) (width 0.25) (layer "F.Cu") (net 3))
 (segment (start 93.599 87.757) (end 91.356 90) (width 0.25) (layer "F.Cu") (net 3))
 (segment (start 93.599 82.5754) (end 93.599 87.757) (width 0.25) (layer "F.Cu") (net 3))
 (segment (start 95.4794 80.695) (end 93.599 82.5754) (width 0.25) (layer "F.Cu") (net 3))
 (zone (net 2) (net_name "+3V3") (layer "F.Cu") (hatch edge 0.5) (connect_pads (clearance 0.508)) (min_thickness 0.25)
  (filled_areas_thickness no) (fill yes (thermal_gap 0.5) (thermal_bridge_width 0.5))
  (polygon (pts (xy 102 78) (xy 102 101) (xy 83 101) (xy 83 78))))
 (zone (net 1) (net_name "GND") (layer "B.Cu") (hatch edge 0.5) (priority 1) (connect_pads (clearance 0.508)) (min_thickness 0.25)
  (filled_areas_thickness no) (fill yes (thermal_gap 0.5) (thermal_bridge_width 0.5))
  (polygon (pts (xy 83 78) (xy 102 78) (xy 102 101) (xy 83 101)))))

